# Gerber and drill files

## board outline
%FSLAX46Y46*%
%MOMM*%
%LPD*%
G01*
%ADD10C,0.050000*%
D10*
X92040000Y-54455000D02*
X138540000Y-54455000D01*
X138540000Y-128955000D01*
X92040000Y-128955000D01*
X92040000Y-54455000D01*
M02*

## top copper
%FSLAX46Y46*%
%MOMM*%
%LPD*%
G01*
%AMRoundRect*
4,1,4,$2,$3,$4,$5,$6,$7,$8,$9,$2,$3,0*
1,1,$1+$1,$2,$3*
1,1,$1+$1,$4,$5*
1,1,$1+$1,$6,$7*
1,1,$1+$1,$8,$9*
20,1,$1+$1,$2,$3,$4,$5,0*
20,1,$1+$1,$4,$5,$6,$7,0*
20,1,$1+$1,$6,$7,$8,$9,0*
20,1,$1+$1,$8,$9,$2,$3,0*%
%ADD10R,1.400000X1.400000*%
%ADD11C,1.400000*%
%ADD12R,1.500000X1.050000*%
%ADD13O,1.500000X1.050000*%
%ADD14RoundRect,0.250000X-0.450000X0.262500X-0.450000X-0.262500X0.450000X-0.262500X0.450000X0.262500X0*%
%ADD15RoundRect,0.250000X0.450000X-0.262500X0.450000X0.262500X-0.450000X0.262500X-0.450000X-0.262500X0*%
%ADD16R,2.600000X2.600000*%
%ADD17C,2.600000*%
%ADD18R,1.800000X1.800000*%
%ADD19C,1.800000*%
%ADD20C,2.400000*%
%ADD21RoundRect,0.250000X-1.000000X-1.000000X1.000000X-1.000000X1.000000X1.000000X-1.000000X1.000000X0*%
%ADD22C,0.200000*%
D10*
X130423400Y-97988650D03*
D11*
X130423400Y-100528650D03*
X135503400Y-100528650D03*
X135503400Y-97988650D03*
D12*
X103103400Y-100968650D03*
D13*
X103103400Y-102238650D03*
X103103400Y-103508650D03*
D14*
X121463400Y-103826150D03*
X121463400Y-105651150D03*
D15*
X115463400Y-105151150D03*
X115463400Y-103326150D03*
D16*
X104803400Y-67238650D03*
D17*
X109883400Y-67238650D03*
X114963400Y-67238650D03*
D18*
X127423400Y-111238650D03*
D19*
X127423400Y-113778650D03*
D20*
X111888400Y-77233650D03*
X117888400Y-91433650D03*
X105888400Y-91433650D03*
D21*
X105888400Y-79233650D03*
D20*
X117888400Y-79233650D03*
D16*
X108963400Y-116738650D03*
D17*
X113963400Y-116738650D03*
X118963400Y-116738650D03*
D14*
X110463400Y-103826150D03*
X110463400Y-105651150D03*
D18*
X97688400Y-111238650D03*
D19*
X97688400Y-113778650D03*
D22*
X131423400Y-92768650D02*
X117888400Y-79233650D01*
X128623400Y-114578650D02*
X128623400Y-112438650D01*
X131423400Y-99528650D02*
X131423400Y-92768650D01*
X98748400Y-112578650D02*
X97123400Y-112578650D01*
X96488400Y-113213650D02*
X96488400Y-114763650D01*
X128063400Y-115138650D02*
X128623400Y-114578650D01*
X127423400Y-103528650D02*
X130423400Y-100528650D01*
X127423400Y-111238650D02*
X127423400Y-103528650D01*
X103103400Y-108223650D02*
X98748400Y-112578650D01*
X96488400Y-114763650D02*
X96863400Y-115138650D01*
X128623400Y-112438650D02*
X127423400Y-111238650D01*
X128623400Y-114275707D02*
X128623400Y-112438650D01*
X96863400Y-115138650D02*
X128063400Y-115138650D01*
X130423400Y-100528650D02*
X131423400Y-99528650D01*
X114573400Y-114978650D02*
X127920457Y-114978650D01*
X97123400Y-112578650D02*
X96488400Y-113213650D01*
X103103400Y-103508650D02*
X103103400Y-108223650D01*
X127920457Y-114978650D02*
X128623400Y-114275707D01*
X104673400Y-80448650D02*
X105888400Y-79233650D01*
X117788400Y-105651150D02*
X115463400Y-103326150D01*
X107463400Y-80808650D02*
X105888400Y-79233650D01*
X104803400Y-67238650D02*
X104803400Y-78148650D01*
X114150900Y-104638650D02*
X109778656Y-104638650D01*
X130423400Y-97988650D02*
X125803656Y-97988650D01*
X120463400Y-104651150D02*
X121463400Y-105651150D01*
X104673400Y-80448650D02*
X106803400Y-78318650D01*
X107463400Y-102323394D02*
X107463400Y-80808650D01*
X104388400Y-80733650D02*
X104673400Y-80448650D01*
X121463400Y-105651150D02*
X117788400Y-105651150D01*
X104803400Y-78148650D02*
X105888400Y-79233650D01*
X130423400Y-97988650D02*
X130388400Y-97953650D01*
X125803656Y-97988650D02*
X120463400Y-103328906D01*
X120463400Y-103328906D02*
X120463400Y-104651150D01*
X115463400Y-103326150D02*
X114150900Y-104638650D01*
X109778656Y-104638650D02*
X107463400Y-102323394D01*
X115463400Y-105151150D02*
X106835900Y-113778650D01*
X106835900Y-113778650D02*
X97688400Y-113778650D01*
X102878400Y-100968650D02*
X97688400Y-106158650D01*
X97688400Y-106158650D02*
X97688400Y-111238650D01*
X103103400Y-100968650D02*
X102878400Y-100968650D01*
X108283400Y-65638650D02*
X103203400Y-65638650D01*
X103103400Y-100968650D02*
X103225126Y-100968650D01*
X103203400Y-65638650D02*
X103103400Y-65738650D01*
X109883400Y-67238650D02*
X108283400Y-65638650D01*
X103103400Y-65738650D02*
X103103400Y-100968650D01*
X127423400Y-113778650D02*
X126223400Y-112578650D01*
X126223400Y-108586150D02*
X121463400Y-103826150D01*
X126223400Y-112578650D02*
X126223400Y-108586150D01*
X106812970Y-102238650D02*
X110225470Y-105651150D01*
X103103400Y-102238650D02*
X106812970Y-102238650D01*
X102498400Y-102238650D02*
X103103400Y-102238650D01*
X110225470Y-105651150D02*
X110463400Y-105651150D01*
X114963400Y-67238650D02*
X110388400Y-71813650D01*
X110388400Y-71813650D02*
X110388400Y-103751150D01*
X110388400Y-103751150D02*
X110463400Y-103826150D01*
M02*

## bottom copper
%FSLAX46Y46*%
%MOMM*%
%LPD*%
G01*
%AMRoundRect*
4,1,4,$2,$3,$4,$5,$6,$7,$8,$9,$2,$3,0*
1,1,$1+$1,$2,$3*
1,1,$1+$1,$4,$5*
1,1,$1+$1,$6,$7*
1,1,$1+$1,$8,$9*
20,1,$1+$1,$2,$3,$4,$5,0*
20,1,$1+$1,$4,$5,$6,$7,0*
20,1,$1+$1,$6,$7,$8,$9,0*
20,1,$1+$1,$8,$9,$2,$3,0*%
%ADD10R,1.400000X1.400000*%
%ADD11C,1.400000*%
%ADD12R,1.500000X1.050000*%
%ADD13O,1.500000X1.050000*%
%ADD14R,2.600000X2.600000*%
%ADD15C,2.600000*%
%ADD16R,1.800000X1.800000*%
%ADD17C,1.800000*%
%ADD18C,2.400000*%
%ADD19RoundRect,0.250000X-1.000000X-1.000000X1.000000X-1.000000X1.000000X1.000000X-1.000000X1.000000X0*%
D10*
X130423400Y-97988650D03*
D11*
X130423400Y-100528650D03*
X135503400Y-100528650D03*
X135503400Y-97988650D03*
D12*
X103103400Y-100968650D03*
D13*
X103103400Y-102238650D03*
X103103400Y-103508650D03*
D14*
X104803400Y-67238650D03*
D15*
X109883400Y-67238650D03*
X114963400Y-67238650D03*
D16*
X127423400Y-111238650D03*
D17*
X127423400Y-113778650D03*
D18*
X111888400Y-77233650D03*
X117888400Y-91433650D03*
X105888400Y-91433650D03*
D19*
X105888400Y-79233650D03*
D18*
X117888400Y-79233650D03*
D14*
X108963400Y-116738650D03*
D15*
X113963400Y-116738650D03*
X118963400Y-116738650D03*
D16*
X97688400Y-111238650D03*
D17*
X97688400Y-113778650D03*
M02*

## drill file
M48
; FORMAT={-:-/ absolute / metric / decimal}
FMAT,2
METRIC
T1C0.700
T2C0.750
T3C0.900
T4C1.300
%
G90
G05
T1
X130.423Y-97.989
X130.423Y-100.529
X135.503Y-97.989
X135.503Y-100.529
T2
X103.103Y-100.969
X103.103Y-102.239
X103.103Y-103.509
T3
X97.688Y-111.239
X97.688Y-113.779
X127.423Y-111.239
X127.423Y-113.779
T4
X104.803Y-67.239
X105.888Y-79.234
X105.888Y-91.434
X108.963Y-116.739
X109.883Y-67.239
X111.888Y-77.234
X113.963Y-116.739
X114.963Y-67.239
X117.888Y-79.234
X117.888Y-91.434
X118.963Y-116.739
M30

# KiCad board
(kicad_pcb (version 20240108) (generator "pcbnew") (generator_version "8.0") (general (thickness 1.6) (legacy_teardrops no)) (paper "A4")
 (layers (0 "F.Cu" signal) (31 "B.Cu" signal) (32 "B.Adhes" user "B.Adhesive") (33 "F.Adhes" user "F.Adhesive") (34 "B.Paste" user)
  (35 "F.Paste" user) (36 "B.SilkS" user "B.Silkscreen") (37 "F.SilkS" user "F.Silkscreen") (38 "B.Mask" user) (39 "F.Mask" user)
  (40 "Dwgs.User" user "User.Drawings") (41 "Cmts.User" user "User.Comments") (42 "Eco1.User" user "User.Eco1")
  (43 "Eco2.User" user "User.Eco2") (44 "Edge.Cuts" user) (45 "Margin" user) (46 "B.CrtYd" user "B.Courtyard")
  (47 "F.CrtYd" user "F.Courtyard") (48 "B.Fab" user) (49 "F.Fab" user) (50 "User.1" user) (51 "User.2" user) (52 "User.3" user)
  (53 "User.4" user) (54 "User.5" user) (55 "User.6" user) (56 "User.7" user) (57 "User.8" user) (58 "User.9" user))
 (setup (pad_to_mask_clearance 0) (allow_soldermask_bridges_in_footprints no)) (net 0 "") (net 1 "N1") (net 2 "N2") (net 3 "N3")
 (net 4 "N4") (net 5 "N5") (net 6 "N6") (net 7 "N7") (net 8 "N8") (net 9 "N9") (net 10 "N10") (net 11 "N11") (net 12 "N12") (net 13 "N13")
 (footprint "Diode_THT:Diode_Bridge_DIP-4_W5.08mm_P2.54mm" (layer "F.Cu") (at 130.4234 97.98865)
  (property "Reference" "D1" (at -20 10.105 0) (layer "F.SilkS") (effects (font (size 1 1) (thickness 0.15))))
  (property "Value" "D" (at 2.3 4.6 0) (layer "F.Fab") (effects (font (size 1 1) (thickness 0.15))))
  (pad "1" thru_hole rect (at 0 0) (size 1.4 1.4) (drill 0.7) (layers "*.Cu" "*.Mask") (remove_unused_layers no) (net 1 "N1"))
  (pad "2" thru_hole circle (at 0 2.54) (size 1.4 1.4) (drill 0.7) (layers "*.Cu" "*.Mask") (remove_unused_layers no) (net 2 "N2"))
  (pad "3" thru_hole circle (at 5.08 2.54) (size 1.4 1.4) (drill 0.7) (layers "*.Cu" "*.Mask") (remove_unused_layers no))
  (pad "4" thru_hole circle (at 5.08 0) (size 1.4 1.4) (drill 0.7) (layers "*.Cu" "*.Mask") (remove_unused_layers no)))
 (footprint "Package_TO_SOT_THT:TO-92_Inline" (layer "F.Cu") (at 103.1034 100.96865 -90)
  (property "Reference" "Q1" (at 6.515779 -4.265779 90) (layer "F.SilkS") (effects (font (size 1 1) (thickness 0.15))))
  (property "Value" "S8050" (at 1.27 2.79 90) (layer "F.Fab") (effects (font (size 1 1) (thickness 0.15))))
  (pad "1" thru_hole rect (at 0 0 270) (size 1.05 1.5) (drill 0.75) (layers "*.Cu" "*.Mask") (remove_unused_layers no) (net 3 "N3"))
  (pad "2" thru_hole oval (at 1.27 0 270) (size 1.05 1.5) (drill 0.75) (layers "*.Cu" "*.Mask") (remove_unused_layers no) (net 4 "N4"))
  (pad "3" thru_hole oval (at 2.54 0 270) (size 1.05 1.5) (drill 0.75) (layers "*.Cu" "*.Mask") (remove_unused_layers no) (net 2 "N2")))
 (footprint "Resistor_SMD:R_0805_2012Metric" (layer "F.Cu") (at 121.4634 104.73865 -90)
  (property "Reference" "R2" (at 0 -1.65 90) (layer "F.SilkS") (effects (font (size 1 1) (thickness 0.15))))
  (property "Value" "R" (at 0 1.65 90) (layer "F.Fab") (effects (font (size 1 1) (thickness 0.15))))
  (pad "1" smd roundrect (at -0.9125 0 270) (size 1.025 1.4) (layers "F.Cu" "F.Paste" "F.Mask") (roundrect_rratio 0.243902) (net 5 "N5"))
  (pad "2" smd roundrect (at 0.9125 0 270) (size 1.025 1.4) (layers "F.Cu" "F.Paste" "F.Mask") (roundrect_rratio 0.243902) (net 1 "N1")))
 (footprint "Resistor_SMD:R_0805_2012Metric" (layer "F.Cu") (at 115.4634 104.23865 90)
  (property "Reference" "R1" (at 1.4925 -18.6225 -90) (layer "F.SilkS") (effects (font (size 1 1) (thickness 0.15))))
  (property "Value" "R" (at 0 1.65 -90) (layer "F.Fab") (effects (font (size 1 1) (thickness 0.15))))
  (pad "1" smd roundrect (at -0.9125 0 90) (size 1.025 1.4) (layers "F.Cu" "F.Paste" "F.Mask") (roundrect_rratio 0.243902) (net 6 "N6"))
  (pad "2" smd roundrect (at 0.9125 0 90) (size 1.025 1.4) (layers "F.Cu" "F.Paste" "F.Mask") (roundrect_rratio 0.243902) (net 1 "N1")))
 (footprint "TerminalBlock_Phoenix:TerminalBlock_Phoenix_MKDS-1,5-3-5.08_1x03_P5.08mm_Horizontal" (layer "F.Cu") (at 104.8034 67.23865)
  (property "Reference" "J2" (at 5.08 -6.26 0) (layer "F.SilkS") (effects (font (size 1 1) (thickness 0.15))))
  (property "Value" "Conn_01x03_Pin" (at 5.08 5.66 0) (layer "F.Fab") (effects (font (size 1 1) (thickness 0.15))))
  (pad "1" thru_hole rect (at 0 0) (size 2.6 2.6) (drill 1.3) (layers "*.Cu" "*.Mask") (remove_unused_layers no) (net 1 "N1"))
  (pad "2" thru_hole circle (at 5.08 0) (size 2.6 2.6) (drill 1.3) (layers "*.Cu" "*.Mask") (remove_unused_layers no) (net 3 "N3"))
  (pad "3" thru_hole circle (at 10.16 0) (size 2.6 2.6) (drill 1.3) (layers "*.Cu" "*.Mask") (remove_unused_layers no) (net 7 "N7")))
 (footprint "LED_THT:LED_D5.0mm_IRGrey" (layer "F.Cu") (at 127.4234 111.23865 -90)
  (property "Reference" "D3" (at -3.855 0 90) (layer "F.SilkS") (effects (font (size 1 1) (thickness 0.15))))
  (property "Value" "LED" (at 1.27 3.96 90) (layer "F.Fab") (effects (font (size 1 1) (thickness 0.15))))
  (pad "1" thru_hole rect (at 0 0 270) (size 1.8 1.8) (drill 0.9) (layers "*.Cu" "*.Mask") (remove_unused_layers no) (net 2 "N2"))
  (pad "2" thru_hole circle (at 2.54 0 270) (size 1.8 1.8) (drill 0.9) (layers "*.Cu" "*.Mask") (remove_unused_layers no) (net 5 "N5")))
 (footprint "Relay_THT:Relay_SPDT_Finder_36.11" (layer "F.Cu") (at 105.8884 79.23365)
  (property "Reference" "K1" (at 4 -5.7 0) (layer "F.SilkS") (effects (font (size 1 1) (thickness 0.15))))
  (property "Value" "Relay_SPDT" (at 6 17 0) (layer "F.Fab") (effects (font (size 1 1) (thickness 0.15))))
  (pad "11" thru_hole circle (at 6 -2) (size 2.4 2.4) (drill 1.3) (layers "*.Cu" "*.Mask") (remove_unused_layers no) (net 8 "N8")
   (clearance 0.2))
  (pad "12" thru_hole circle (at 12 12.2) (size 2.4 2.4) (drill 1.3) (layers "*.Cu" "*.Mask") (remove_unused_layers no) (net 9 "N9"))
  (pad "14" thru_hole circle (at 0 12.2) (size 2.4 2.4) (drill 1.3) (layers "*.Cu" "*.Mask") (remove_unused_layers no) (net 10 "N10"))
  (pad "A1" thru_hole roundrect (at 0 0) (size 2.5 2.5) (drill 1.3) (layers "*.Cu" "*.Mask") (remove_unused_layers no)
   (roundrect_rratio 0.1) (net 1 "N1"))
  (pad "A2" thru_hole circle (at 12 0) (size 2.4 2.4) (drill 1.3) (layers "*.Cu" "*.Mask") (remove_unused_layers no) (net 2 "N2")))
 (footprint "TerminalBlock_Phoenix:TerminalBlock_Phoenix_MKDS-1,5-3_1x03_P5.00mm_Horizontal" (layer "F.Cu") (at 108.9634 116.73865)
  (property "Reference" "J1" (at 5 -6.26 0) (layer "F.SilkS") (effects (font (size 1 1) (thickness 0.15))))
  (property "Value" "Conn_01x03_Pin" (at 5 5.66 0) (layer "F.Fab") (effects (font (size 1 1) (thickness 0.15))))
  (pad "1" thru_hole rect (at 0 0) (size 2.6 2.6) (drill 1.3) (layers "*.Cu" "*.Mask") (remove_unused_layers no) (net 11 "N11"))
  (pad "2" thru_hole circle (at 5 0) (size 2.6 2.6) (drill 1.3) (layers "*.Cu" "*.Mask") (remove_unused_layers no) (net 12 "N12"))
  (pad "3" thru_hole circle (at 10 0) (size 2.6 2.6) (drill 1.3) (layers "*.Cu" "*.Mask") (remove_unused_layers no) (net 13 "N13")))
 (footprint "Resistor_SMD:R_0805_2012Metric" (layer "F.Cu") (at 110.4634 104.73865 -90)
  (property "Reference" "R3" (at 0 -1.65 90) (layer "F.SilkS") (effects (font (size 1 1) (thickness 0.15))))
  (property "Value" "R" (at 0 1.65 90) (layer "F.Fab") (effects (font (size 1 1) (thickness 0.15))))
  (pad "1" smd roundrect (at -0.9125 0 270) (size 1.025 1.4) (layers "F.Cu" "F.Paste" "F.Mask") (roundrect_rratio 0.243902) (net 7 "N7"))
  (pad "2" smd roundrect (at 0.9125 0 270) (size 1.025 1.4) (layers "F.Cu" "F.Paste" "F.Mask") (roundrect_rratio 0.243902) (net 4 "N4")))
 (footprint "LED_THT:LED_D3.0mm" (layer "F.Cu") (at 97.6884 111.23865 -90)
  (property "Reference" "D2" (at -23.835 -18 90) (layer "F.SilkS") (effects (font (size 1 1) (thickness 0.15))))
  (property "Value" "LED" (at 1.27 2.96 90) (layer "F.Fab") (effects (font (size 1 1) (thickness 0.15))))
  (pad "1" thru_hole rect (at 0 0 270) (size 1.8 1.8) (drill 0.9) (layers "*.Cu" "*.Mask") (remove_unused_layers no) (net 3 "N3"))
  (pad "2" thru_hole circle (at 2.54 0 270) (size 1.8 1.8) (drill 0.9) (layers "*.Cu" "*.Mask") (remove_unused_layers no) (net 6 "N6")))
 (gr_rect (start 92.04 54.455) (end 138.54 128.955) (stroke (width 0.05) (type default)) (fill none) (layer "Edge.Cuts"))
 (segment (start 131.4234 92.76865) (end 117.8884 79.23365) (width 0.2) (layer "F.Cu") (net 2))
 (segment (start 128.6234 114.57865) (end 128.6234 112.43865) (width 0.2) (layer "F.Cu") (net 2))
 (segment (start 131.4234 99.52865) (end 131.4234 92.76865) (width 0.2) (layer "F.Cu") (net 2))
 (segment (start 98.7484 112.57865) (end 97.1234 112.57865) (width 0.2) (layer "F.Cu") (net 2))
 (segment (start 96.4884 113.21365) (end 96.4884 114.76365) (width 0.2) (layer "F.Cu") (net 2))
 (segment (start 128.0634 115.13865) (end 128.6234 114.57865) (width 0.2) (layer "F.Cu") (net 2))
 (segment (start 127.4234 103.52865) (end 130.4234 100.52865) (width 0.2) (layer "F.Cu") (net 2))
 (segment (start 127.4234 111.23865) (end 127.4234 103.52865) (width 0.2) (layer "F.Cu") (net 2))
 (segment (start 103.1034 108.22365) (end 98.7484 112.57865) (width 0.2) (layer "F.Cu") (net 2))
 (segment (start 96.4884 114.76365) (end 96.8634 115.13865) (width 0.2) (layer "F.Cu") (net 2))
 (segment (start 128.6234 112.43865) (end 127.4234 111.23865) (width 0.2) (layer "F.Cu") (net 2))
 (segment (start 128.6234 114.275707) (end 128.6234 112.43865) (width 0.2) (layer "F.Cu") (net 2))
 (segment (start 96.8634 115.13865) (end 128.0634 115.13865) (width 0.2) (layer "F.Cu") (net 2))
 (segment (start 130.4234 100.52865) (end 131.4234 99.52865) (width 0.2) (layer "F.Cu") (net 2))
 (segment (start 114.5734 114.97865) (end 127.920457 114.97865) (width 0.2) (layer "F.Cu") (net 2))
 (segment (start 97.1234 112.57865) (end 96.4884 113.21365) (width 0.2) (layer "F.Cu") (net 2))
 (segment (start 103.1034 103.50865) (end 103.1034 108.22365) (width 0.2) (layer "F.Cu") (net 2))
 (segment (start 127.920457 114.97865) (end 128.6234 114.275707) (width 0.2) (layer "F.Cu") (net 2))
 (segment (start 104.6734 80.44865) (end 105.8884 79.23365) (width 0.2) (layer "F.Cu") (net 1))
 (segment (start 117.7884 105.65115) (end 115.4634 103.32615) (width 0.2) (layer "F.Cu") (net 1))
 (segment (start 107.4634 80.80865) (end 105.8884 79.23365) (width 0.2) (layer "F.Cu") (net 1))
 (segment (start 104.8034 67.23865) (end 104.8034 78.14865) (width 0.2) (layer "F.Cu") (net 1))
 (segment (start 114.1509 104.63865) (end 109.778656 104.63865) (width 0.2) (layer "F.Cu") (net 1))
 (segment (start 130.4234 97.98865) (end 125.803656 97.98865) (width 0.2) (layer "F.Cu") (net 1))
 (segment (start 120.4634 104.65115) (end 121.4634 105.65115) (width 0.2) (layer "F.Cu") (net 1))
 (segment (start 104.6734 80.44865) (end 106.8034 78.31865) (width 0.2) (layer "F.Cu") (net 1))
 (segment (start 107.4634 102.323394) (end 107.4634 80.80865) (width 0.2) (layer "F.Cu") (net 1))
 (segment (start 104.3884 80.73365) (end 104.6734 80.44865) (width 0.2) (layer "F.Cu") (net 1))
 (segment (start 121.4634 105.65115) (end 117.7884 105.65115) (width 0.2) (layer "F.Cu") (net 1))
 (segment (start 104.8034 78.14865) (end 105.8884 79.23365) (width 0.2) (layer "F.Cu") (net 1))
 (segment (start 130.4234 97.98865) (end 130.3884 97.95365) (width 0.2) (layer "F.Cu") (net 1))
 (segment (start 125.803656 97.98865) (end 120.4634 103.328906) (width 0.2) (layer "F.Cu") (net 1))
 (segment (start 120.4634 103.328906) (end 120.4634 104.65115) (width 0.2) (layer "F.Cu") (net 1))
 (segment (start 115.4634 103.32615) (end 114.1509 104.63865) (width 0.2) (layer "F.Cu") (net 1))
 (segment (start 109.778656 104.63865) (end 107.4634 102.323394) (width 0.2) (layer "F.Cu") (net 1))
 (segment (start 115.4634 105.15115) (end 106.8359 113.77865) (width 0.2) (layer "F.Cu") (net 6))
 (segment (start 106.8359 113.77865) (end 97.6884 113.77865) (width 0.2) (layer "F.Cu") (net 6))
 (segment (start 102.8784 100.96865) (end 97.6884 106.15865) (width 0.2) (layer "F.Cu") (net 3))
 (segment (start 97.6884 106.15865) (end 97.6884 111.23865) (width 0.2) (layer "F.Cu") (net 3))
 (segment (start 103.1034 100.96865) (end 102.8784 100.96865) (width 0.2) (layer "F.Cu") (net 3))
 (segment (start 108.2834 65.63865) (end 103.2034 65.63865) (width 0.2) (layer "F.Cu") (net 3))
 (segment (start 103.1034 100.96865) (end 103.225126 100.96865) (width 0.2) (layer "F.Cu") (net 3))
 (segment (start 103.2034 65.63865) (end 103.1034 65.73865) (width 0.2) (layer "F.Cu") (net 3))
 (segment (start 109.8834 67.23865) (end 108.2834 65.63865) (width 0.2) (layer "F.Cu") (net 3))
 (segment (start 103.1034 65.73865) (end 103.1034 100.96865) (width 0.2) (layer "F.Cu") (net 3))
 (segment (start 127.4234 113.77865) (end 126.2234 112.57865) (width 0.2) (layer "F.Cu") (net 5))
 (segment (start 126.2234 108.58615) (end 121.4634 103.82615) (width 0.2) (layer "F.Cu") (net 5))
 (segment (start 126.2234 112.57865) (end 126.2234 108.58615) (width 0.2) (layer "F.Cu") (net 5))
 (segment (start 106.81297 102.23865) (end 110.22547 105.65115) (width 0.2) (layer "F.Cu") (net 4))
 (segment (start 103.1034 102.23865) (end 106.81297 102.23865) (width 0.2) (layer "F.Cu") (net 4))
 (segment (start 102.4984 102.23865) (end 103.1034 102.23865) (width 0.2) (layer "F.Cu") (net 4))
 (segment (start 110.22547 105.65115) (end 110.4634 105.65115) (width 0.2) (layer "F.Cu") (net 4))
 (segment (start 114.9634 67.23865) (end 110.3884 71.81365) (width 0.2) (layer "F.Cu") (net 7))
 (segment (start 110.3884 71.81365) (end 110.3884 103.75115) (width 0.2) (layer "F.Cu") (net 7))
 (segment (start 110.3884 103.75115) (end 110.4634 103.82615) (width 0.2) (layer "F.Cu") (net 7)))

